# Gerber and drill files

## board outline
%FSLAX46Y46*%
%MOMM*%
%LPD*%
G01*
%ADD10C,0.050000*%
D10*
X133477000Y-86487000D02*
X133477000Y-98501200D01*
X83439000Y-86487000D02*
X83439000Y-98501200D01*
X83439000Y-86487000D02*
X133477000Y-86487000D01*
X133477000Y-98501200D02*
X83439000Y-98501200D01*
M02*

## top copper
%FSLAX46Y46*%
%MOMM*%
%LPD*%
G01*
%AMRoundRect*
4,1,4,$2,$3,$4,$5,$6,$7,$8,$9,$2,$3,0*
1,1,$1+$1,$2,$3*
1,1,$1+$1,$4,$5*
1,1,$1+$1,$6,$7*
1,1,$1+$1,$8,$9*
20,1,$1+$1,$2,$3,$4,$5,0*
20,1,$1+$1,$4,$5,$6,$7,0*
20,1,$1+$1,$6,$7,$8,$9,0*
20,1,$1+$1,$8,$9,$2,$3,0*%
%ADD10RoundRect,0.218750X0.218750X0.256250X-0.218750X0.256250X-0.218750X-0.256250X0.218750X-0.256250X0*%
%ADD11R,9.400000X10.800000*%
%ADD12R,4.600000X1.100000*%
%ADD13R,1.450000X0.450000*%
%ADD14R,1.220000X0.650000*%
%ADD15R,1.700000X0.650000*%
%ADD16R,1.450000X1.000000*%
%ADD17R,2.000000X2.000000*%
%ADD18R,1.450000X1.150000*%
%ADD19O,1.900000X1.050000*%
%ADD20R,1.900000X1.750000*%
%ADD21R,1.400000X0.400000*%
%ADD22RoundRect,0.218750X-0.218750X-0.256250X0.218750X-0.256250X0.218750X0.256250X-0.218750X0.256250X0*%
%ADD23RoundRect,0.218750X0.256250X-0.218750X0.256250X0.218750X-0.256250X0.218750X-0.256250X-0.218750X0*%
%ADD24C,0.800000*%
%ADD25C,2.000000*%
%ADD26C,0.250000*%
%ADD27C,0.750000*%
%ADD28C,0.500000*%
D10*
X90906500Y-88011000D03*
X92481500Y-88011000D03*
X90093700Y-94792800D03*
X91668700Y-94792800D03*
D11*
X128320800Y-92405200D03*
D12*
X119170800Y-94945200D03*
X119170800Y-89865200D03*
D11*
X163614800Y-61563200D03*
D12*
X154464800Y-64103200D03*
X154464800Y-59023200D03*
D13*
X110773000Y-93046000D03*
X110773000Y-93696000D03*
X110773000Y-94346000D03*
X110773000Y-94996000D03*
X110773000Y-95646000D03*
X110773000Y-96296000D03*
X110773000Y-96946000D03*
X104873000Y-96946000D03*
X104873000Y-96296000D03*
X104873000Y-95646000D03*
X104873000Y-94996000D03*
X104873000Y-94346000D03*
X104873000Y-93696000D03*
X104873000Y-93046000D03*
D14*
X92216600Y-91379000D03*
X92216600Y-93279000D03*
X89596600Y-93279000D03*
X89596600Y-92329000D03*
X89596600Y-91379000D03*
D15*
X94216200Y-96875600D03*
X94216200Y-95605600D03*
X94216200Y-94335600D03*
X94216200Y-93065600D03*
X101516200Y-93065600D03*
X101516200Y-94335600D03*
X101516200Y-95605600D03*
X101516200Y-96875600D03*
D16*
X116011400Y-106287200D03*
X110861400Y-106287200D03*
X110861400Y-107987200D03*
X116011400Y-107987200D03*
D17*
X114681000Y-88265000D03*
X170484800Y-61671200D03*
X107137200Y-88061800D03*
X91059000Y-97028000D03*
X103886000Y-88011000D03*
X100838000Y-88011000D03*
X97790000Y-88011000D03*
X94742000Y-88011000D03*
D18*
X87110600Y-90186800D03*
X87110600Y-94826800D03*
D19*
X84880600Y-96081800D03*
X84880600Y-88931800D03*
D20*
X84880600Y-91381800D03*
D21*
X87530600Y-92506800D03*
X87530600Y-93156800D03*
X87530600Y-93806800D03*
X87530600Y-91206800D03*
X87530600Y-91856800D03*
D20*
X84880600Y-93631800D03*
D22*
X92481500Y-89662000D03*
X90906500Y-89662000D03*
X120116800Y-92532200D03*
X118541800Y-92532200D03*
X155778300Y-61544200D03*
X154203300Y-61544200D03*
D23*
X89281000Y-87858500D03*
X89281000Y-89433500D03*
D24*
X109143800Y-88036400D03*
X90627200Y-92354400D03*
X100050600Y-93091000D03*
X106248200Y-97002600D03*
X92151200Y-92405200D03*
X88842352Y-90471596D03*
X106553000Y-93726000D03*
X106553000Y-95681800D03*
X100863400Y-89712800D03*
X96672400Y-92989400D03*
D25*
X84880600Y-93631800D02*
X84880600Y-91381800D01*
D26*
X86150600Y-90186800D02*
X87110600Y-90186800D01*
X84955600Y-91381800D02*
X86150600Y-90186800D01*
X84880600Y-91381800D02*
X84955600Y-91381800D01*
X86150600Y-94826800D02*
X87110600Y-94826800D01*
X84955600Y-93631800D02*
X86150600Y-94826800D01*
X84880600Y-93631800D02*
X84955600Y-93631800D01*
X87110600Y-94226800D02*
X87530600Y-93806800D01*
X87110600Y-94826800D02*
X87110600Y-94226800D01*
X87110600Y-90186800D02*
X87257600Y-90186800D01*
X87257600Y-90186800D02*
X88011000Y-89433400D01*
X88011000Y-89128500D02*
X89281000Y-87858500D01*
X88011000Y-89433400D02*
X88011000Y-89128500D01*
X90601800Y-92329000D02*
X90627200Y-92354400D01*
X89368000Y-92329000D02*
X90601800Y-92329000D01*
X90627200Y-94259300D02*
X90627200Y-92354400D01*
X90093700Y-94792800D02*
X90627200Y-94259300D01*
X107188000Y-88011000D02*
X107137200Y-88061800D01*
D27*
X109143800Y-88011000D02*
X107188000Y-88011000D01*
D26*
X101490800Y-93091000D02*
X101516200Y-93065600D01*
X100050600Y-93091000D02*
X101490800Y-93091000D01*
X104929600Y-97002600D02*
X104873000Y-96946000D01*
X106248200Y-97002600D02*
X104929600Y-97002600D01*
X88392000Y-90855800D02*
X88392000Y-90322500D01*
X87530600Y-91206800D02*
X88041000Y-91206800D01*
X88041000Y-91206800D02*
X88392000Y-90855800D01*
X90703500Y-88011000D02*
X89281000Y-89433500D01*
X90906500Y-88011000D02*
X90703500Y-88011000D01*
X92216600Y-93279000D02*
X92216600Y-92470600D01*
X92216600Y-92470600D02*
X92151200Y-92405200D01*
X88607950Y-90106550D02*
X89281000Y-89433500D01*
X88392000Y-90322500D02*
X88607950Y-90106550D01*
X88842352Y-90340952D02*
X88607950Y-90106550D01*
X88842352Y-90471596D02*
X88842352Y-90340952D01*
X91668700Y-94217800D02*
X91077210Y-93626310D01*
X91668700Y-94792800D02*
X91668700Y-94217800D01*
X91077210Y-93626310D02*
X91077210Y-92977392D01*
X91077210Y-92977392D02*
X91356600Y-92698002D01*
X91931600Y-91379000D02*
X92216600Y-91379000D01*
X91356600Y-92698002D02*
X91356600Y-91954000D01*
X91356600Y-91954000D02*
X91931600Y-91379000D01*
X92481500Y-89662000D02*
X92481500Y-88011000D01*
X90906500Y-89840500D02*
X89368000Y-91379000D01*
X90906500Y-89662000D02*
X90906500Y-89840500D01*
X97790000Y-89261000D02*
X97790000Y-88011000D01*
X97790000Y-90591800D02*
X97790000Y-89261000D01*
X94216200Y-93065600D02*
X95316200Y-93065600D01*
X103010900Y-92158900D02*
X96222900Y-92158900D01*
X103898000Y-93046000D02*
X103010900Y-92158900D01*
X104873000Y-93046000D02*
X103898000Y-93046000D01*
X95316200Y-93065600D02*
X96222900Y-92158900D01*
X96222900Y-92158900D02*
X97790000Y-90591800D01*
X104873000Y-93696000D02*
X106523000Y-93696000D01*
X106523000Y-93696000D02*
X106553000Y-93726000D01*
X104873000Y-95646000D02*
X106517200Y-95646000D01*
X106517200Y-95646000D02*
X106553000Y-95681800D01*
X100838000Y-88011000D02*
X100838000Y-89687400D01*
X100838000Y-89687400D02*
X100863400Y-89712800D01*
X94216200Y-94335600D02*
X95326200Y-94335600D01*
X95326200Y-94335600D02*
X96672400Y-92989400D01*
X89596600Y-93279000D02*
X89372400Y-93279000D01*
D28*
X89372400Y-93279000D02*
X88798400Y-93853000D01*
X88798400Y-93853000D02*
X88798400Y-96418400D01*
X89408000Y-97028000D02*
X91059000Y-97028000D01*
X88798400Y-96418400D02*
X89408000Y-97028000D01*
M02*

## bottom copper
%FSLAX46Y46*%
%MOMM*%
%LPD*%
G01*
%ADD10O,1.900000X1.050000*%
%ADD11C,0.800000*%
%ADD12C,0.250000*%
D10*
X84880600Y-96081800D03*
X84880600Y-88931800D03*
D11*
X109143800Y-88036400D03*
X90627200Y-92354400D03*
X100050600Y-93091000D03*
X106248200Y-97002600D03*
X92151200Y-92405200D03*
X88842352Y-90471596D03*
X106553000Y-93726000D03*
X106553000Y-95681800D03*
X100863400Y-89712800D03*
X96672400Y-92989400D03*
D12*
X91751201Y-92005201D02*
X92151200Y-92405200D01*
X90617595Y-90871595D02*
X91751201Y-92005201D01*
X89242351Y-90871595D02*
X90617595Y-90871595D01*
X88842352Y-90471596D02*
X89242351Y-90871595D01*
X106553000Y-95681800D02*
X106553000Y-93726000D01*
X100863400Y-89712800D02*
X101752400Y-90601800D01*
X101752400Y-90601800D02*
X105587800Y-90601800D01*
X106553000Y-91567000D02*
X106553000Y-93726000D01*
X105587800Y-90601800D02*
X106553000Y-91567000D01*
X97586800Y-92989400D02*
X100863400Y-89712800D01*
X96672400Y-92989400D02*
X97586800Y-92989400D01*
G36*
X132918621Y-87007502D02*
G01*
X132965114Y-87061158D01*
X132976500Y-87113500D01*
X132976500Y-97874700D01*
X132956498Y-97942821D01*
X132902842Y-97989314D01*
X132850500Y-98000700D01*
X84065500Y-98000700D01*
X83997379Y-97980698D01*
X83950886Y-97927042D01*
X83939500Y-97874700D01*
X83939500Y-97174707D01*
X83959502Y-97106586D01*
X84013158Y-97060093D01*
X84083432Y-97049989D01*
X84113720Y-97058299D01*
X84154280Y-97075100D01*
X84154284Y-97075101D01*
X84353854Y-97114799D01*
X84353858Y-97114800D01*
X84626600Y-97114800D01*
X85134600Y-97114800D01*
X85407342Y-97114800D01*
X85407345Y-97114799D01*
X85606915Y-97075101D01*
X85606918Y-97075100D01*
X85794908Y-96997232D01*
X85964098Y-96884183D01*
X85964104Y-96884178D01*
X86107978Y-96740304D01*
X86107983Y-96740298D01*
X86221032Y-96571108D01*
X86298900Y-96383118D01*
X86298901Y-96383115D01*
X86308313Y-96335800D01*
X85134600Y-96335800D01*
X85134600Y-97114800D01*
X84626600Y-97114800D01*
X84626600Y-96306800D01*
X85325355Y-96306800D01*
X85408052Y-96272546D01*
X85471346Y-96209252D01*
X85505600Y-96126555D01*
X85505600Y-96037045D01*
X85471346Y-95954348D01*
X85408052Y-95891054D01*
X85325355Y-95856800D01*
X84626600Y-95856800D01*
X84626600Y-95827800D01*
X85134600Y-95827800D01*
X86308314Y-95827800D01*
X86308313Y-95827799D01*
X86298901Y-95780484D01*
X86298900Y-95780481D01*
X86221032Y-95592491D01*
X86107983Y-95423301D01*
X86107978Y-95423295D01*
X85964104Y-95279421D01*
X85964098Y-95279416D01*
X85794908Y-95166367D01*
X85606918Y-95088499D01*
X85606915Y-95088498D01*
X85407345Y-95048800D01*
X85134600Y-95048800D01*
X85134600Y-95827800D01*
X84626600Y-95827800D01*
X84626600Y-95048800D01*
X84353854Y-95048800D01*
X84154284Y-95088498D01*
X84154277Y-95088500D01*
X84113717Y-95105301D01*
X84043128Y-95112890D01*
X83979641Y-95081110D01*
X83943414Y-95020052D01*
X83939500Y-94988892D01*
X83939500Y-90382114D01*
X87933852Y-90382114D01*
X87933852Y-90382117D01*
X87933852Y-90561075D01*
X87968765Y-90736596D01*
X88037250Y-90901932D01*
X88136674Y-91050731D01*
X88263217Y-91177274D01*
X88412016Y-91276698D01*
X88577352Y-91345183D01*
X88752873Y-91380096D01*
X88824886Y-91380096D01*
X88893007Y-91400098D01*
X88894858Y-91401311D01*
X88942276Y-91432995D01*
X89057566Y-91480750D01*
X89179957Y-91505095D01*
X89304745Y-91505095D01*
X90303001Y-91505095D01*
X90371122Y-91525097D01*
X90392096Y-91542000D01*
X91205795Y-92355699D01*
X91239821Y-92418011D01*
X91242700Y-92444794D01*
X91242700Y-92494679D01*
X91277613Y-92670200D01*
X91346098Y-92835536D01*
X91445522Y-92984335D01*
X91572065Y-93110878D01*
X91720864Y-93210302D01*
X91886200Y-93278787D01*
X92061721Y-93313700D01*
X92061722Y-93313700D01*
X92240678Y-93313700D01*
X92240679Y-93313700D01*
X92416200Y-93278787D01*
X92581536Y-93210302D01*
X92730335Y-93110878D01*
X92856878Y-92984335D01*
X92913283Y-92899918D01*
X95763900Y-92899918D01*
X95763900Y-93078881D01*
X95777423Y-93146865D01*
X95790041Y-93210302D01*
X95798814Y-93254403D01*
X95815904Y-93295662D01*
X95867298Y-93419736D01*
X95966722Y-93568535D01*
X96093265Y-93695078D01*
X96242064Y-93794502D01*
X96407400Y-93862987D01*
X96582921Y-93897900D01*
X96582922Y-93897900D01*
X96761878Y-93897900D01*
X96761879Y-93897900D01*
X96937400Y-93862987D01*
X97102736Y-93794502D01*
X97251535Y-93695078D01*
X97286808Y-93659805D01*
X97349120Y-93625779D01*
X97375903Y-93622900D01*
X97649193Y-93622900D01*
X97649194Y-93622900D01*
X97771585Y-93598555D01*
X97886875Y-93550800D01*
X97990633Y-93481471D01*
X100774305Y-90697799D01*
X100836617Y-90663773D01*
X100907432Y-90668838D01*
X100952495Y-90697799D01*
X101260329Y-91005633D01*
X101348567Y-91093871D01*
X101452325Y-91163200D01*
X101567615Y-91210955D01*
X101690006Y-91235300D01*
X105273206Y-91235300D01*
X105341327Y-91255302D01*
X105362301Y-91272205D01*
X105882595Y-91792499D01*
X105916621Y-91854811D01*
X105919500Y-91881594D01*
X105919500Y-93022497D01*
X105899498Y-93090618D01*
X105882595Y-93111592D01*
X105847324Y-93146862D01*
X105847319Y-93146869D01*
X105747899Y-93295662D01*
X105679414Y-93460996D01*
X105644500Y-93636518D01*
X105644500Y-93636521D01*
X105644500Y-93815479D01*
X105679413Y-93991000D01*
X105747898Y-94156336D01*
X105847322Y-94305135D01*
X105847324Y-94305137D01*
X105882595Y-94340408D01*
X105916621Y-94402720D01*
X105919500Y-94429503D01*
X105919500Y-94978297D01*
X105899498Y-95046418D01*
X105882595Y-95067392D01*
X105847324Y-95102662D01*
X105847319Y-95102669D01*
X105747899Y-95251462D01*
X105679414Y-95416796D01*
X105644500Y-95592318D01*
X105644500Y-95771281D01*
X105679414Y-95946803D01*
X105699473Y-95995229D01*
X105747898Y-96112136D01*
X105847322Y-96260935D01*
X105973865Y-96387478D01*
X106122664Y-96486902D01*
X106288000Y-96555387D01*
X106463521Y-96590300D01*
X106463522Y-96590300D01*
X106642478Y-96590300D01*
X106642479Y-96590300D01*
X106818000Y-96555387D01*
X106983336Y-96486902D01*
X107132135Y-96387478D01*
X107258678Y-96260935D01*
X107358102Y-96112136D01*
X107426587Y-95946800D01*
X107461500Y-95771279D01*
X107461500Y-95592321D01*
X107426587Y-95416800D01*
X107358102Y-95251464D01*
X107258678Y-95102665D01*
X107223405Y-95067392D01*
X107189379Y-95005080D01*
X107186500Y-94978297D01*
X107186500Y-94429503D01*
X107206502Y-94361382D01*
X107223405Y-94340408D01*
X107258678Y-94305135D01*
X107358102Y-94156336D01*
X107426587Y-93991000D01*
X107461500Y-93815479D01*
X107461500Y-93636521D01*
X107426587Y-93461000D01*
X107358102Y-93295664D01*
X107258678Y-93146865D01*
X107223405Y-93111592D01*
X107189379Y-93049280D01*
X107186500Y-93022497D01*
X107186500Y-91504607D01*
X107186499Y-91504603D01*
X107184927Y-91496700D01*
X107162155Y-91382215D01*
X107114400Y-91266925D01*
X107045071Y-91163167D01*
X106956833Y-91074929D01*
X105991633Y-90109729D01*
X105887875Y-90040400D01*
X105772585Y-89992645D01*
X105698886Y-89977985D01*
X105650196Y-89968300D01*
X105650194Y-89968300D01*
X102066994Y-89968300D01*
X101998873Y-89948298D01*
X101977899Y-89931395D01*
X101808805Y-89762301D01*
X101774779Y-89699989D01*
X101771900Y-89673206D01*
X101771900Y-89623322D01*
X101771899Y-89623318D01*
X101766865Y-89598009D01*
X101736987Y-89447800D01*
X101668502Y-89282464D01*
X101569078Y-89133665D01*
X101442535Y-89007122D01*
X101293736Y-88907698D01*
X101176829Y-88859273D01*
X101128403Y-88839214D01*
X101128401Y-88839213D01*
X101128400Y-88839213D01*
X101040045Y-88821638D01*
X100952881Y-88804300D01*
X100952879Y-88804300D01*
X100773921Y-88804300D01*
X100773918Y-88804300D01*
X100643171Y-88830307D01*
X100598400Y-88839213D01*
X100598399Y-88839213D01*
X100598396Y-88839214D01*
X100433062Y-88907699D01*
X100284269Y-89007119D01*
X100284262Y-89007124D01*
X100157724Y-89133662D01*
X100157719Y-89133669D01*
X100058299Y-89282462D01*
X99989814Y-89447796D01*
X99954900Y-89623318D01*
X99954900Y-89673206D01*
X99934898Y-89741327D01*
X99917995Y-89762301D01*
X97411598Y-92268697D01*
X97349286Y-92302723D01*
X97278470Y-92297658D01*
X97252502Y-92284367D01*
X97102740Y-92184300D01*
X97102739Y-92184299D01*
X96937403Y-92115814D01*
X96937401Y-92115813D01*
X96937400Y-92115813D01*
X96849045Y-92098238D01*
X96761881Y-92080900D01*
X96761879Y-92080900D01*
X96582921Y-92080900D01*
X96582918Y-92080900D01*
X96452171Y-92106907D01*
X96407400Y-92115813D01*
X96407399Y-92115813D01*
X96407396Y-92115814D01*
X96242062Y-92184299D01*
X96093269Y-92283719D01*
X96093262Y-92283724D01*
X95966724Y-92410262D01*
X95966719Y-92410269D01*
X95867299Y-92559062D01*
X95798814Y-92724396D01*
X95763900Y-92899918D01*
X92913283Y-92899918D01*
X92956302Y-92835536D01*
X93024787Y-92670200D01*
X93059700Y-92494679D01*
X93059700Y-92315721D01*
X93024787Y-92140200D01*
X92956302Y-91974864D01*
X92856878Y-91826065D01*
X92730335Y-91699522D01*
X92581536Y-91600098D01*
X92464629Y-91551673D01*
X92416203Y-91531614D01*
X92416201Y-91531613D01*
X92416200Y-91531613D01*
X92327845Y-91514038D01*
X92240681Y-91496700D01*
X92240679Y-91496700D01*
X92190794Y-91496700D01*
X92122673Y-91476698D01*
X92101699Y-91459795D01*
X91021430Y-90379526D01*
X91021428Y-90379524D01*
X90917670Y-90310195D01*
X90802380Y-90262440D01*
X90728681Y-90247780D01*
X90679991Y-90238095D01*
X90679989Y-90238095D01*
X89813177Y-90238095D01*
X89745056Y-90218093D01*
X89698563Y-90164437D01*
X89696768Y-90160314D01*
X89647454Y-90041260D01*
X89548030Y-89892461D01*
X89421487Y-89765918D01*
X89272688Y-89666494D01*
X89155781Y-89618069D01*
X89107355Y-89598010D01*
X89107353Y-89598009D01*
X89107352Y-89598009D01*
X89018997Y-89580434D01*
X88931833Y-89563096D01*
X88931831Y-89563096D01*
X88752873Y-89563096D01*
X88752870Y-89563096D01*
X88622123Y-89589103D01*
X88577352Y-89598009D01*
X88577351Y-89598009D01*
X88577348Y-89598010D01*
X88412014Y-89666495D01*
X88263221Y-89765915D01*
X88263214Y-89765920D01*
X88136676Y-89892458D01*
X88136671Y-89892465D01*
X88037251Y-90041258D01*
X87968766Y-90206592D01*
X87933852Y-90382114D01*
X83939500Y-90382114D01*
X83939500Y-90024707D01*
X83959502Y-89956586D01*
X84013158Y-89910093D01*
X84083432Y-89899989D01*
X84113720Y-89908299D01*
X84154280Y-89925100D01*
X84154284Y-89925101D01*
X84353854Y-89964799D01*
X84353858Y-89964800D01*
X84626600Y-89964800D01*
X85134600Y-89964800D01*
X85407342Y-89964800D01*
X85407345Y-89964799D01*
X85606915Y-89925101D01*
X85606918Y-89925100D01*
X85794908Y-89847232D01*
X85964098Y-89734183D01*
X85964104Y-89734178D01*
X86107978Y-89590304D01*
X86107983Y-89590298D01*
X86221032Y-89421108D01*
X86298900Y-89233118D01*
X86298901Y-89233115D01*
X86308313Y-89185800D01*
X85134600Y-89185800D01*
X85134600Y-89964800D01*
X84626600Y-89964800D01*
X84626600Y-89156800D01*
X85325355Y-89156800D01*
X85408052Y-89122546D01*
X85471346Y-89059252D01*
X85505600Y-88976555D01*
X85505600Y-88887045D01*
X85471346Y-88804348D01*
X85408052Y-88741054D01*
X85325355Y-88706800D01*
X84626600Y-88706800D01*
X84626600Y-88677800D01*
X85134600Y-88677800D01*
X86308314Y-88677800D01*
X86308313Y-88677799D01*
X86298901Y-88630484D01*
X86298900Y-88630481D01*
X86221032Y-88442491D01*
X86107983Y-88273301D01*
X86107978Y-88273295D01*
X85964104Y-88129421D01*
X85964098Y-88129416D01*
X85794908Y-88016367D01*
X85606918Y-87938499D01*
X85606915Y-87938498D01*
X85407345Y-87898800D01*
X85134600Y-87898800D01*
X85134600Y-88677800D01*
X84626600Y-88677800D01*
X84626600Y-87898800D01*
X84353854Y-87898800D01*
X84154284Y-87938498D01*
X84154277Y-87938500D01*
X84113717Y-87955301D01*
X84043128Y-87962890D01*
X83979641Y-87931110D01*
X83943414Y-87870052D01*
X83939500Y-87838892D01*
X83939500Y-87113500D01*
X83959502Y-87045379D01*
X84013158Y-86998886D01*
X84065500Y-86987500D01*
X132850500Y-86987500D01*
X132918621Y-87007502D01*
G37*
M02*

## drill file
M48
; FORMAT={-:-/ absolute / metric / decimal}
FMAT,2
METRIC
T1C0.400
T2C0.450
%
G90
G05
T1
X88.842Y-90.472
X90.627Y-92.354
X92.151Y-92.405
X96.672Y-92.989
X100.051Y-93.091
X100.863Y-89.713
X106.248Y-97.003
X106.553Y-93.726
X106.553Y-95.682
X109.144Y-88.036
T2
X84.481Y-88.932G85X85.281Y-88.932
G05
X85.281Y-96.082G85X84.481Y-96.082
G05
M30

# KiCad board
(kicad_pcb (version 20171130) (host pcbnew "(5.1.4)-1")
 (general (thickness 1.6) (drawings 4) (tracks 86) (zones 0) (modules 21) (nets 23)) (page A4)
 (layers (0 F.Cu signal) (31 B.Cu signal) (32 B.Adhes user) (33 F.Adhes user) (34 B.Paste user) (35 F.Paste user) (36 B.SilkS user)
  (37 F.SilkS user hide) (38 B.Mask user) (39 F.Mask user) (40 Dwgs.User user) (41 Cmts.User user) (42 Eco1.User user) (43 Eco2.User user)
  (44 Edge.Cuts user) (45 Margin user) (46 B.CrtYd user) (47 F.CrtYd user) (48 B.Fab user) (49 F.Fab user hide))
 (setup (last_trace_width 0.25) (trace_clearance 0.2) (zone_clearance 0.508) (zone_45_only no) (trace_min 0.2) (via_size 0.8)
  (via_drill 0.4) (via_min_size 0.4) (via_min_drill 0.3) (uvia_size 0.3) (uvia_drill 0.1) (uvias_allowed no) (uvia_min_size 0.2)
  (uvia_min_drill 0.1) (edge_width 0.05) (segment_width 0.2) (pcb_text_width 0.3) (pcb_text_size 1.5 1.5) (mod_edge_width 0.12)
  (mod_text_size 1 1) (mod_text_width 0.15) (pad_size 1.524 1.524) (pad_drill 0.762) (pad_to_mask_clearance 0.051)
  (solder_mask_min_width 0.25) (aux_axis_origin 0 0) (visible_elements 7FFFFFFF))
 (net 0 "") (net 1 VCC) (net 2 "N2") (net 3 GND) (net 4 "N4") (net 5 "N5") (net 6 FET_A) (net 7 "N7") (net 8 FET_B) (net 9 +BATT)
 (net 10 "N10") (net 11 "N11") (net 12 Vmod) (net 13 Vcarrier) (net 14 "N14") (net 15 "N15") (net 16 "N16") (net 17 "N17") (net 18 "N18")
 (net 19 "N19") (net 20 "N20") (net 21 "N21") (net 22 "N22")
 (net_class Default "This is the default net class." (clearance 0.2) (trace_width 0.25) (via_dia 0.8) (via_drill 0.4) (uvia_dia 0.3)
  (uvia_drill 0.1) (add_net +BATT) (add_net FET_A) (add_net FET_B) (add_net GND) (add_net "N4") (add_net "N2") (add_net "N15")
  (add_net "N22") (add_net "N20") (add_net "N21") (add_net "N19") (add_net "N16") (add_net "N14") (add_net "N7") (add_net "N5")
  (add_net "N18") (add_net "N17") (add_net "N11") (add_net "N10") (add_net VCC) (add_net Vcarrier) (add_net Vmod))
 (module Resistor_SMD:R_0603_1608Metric (layer F.Cu) (at 91.694 88.011 180)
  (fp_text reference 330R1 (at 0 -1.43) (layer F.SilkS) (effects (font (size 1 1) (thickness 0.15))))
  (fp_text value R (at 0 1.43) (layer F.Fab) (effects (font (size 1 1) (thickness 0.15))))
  (pad 2 smd roundrect (at 0.7875 0 180) (size 0.875 0.95) (layers F.Cu F.Paste F.Mask) (roundrect_rratio 0.25) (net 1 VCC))
  (pad 1 smd roundrect (at -0.7875 0 180) (size 0.875 0.95) (layers F.Cu F.Paste F.Mask) (roundrect_rratio 0.25) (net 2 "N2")))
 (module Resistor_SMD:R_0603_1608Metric (layer F.Cu) (at 90.8812 94.7928 180)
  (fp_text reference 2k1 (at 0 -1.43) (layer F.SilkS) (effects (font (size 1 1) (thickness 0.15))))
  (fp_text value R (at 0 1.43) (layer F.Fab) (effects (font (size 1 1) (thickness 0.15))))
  (pad 2 smd roundrect (at 0.7875 0 180) (size 0.875 0.95) (layers F.Cu F.Paste F.Mask) (roundrect_rratio 0.25) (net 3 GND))
  (pad 1 smd roundrect (at -0.7875 0 180) (size 0.875 0.95) (layers F.Cu F.Paste F.Mask) (roundrect_rratio 0.25) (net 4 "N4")))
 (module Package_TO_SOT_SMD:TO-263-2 (layer F.Cu) (at 124.9458 92.4052)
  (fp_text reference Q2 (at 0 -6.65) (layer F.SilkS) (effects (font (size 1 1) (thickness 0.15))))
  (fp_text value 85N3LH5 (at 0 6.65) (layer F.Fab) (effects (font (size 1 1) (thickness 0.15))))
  (pad "" smd rect (at 0.95 2.775) (size 4.55 5.25) (layers F.Paste))
  (pad "" smd rect (at 5.8 -2.775) (size 4.55 5.25) (layers F.Paste))
  (pad "" smd rect (at 0.95 -2.775) (size 4.55 5.25) (layers F.Paste))
  (pad "" smd rect (at 5.8 2.775) (size 4.55 5.25) (layers F.Paste))
  (pad 2 smd rect (at 3.375 0) (size 9.4 10.8) (layers F.Cu F.Mask) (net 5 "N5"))
  (pad 3 smd rect (at -5.775 2.54) (size 4.6 1.1) (layers F.Cu F.Paste F.Mask) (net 3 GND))
  (pad 1 smd rect (at -5.775 -2.54) (size 4.6 1.1) (layers F.Cu F.Paste F.Mask) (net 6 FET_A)))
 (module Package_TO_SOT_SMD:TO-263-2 (layer F.Cu) (at 160.2398 61.5632)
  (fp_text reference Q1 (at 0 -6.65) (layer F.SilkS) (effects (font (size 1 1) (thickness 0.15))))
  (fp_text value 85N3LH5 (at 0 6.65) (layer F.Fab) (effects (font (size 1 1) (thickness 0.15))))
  (pad "" smd rect (at 0.95 2.775) (size 4.55 5.25) (layers F.Paste))
  (pad "" smd rect (at 5.8 -2.775) (size 4.55 5.25) (layers F.Paste))
  (pad "" smd rect (at 0.95 -2.775) (size 4.55 5.25) (layers F.Paste))
  (pad "" smd rect (at 5.8 2.775) (size 4.55 5.25) (layers F.Paste))
  (pad 2 smd rect (at 3.375 0) (size 9.4 10.8) (layers F.Cu F.Mask) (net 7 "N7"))
  (pad 3 smd rect (at -5.775 2.54) (size 4.6 1.1) (layers F.Cu F.Paste F.Mask) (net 3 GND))
  (pad 1 smd rect (at -5.775 -2.54) (size 4.6 1.1) (layers F.Cu F.Paste F.Mask) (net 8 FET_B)))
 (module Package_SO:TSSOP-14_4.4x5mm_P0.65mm (layer F.Cu) (at 107.823 94.996)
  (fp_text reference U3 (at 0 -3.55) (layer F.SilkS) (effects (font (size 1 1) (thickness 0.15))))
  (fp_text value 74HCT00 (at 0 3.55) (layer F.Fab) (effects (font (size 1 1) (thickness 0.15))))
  (pad 14 smd rect (at 2.95 -1.95) (size 1.45 0.45) (layers F.Cu F.Paste F.Mask) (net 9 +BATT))
  (pad 13 smd rect (at 2.95 -1.3) (size 1.45 0.45) (layers F.Cu F.Paste F.Mask) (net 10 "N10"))
  (pad 12 smd rect (at 2.95 -0.65) (size 1.45 0.45) (layers F.Cu F.Paste F.Mask) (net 10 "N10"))
  (pad 11 smd rect (at 2.95 0) (size 1.45 0.45) (layers F.Cu F.Paste F.Mask) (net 8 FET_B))
  (pad 10 smd rect (at 2.95 0.65) (size 1.45 0.45) (layers F.Cu F.Paste F.Mask) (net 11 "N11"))
  (pad 9 smd rect (at 2.95 1.3) (size 1.45 0.45) (layers F.Cu F.Paste F.Mask) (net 11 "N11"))
  (pad 8 smd rect (at 2.95 1.95) (size 1.45 0.45) (layers F.Cu F.Paste F.Mask) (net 6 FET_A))
  (pad 7 smd rect (at -2.95 1.95) (size 1.45 0.45) (layers F.Cu F.Paste F.Mask) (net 3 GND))
  (pad 6 smd rect (at -2.95 1.3) (size 1.45 0.45) (layers F.Cu F.Paste F.Mask) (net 11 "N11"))
  (pad 5 smd rect (at -2.95 0.65) (size 1.45 0.45) (layers F.Cu F.Paste F.Mask) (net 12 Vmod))
  (pad 4 smd rect (at -2.95 0) (size 1.45 0.45) (layers F.Cu F.Paste F.Mask) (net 10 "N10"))
  (pad 3 smd rect (at -2.95 -0.65) (size 1.45 0.45) (layers F.Cu F.Paste F.Mask) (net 10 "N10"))
  (pad 2 smd rect (at -2.95 -1.3) (size 1.45 0.45) (layers F.Cu F.Paste F.Mask) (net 12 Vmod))
  (pad 1 smd rect (at -2.95 -1.95) (size 1.45 0.45) (layers F.Cu F.Paste F.Mask) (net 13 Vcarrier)))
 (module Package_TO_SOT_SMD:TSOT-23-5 (layer F.Cu) (at 90.9066 92.329)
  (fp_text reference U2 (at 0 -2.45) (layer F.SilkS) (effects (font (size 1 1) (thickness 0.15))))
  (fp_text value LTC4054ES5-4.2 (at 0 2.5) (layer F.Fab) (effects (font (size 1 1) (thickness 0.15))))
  (pad 5 smd rect (at 1.31 -0.95) (size 1.22 0.65) (layers F.Cu F.Paste F.Mask) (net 4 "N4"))
  (pad 4 smd rect (at 1.31 0.95) (size 1.22 0.65) (layers F.Cu F.Paste F.Mask) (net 1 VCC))
  (pad 3 smd rect (at -1.31 0.95) (size 1.22 0.65) (layers F.Cu F.Paste F.Mask) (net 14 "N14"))
  (pad 2 smd rect (at -1.31 0) (size 1.22 0.65) (layers F.Cu F.Paste F.Mask) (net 3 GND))
  (pad 1 smd rect (at -1.31 -0.95) (size 1.22 0.65) (layers F.Cu F.Paste F.Mask) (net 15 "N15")))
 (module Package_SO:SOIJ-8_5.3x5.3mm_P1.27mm (layer F.Cu) (at 97.8662 94.9706 180)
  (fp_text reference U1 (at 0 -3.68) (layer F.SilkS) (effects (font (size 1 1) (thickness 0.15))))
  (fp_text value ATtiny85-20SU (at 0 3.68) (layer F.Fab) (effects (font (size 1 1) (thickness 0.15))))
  (pad 8 smd rect (at 3.65 -1.905 180) (size 1.7 0.65) (layers F.Cu F.Paste F.Mask) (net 9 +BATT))
  (pad 7 smd rect (at 3.65 -0.635 180) (size 1.7 0.65) (layers F.Cu F.Paste F.Mask) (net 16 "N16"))
  (pad 6 smd rect (at 3.65 0.635 180) (size 1.7 0.65) (layers F.Cu F.Paste F.Mask) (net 12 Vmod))
  (pad 5 smd rect (at 3.65 1.905 180) (size 1.7 0.65) (layers F.Cu F.Paste F.Mask) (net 13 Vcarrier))
  (pad 4 smd rect (at -3.65 1.905 180) (size 1.7 0.65) (layers F.Cu F.Paste F.Mask) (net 3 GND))
  (pad 3 smd rect (at -3.65 0.635 180) (size 1.7 0.65) (layers F.Cu F.Paste F.Mask) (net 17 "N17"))
  (pad 2 smd rect (at -3.65 -0.635 180) (size 1.7 0.65) (layers F.Cu F.Paste F.Mask) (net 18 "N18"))
  (pad 1 smd rect (at -3.65 -1.905 180) (size 1.7 0.65) (layers F.Cu F.Paste F.Mask) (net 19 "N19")))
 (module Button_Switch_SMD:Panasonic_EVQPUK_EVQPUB (layer F.Cu) (at 113.4364 107.1372)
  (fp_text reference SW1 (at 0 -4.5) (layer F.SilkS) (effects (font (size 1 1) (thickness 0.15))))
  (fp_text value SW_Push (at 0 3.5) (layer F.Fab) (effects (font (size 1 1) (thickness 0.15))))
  (pad 1 smd rect (at 2.575 -0.85 180) (size 1.45 1) (layers F.Cu F.Paste F.Mask) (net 14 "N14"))
  (pad 1 smd rect (at -2.575 -0.85 180) (size 1.45 1) (layers F.Cu F.Paste F.Mask) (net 14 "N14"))
  (pad 2 smd rect (at -2.575 0.85 180) (size 1.45 1) (layers F.Cu F.Paste F.Mask) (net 9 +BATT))
  (pad 2 smd rect (at 2.575 0.85 180) (size 1.45 1) (layers F.Cu F.Paste F.Mask) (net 9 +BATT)))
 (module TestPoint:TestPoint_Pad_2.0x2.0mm (layer F.Cu) (at 114.681 88.265)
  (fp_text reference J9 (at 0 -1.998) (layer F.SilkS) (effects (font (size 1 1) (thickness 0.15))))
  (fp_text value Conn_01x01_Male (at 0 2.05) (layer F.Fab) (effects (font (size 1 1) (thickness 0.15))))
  (pad 1 smd rect (at 0 0) (size 2 2) (layers F.Cu F.Mask) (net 5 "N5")))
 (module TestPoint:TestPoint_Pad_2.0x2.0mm (layer F.Cu) (at 170.4848 61.6712)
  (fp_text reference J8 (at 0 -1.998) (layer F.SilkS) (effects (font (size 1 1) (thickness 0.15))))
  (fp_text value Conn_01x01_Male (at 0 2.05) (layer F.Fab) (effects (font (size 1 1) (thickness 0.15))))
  (pad 1 smd rect (at 0 0) (size 2 2) (layers F.Cu F.Mask) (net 7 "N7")))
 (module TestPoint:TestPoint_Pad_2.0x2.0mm (layer F.Cu) (at 107.1372 88.0618)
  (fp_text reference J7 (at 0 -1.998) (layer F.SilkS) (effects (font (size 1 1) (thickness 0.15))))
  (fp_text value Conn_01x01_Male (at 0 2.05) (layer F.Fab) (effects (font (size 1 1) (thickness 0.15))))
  (pad 1 smd rect (at 0 0) (size 2 2) (layers F.Cu F.Mask) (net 3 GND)))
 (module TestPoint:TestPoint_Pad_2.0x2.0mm (layer F.Cu) (at 91.059 97.028)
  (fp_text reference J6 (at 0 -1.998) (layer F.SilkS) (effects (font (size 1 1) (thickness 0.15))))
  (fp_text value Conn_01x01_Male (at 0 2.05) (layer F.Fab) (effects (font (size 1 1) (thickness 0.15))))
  (pad 1 smd rect (at 0 0) (size 2 2) (layers F.Cu F.Mask) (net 14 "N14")))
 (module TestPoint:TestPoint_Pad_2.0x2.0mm (layer F.Cu) (at 103.886 88.011)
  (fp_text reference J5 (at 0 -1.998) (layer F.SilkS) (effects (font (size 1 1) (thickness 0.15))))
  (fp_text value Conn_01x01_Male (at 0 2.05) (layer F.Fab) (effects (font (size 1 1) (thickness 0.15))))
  (pad 1 smd rect (at 0 0) (size 2 2) (layers F.Cu F.Mask) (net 16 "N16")))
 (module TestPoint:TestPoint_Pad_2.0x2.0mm (layer F.Cu) (at 100.838 88.011)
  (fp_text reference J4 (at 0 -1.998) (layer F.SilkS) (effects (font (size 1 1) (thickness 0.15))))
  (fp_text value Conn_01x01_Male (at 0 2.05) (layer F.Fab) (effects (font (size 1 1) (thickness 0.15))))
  (pad 1 smd rect (at 0 0) (size 2 2) (layers F.Cu F.Mask) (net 12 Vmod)))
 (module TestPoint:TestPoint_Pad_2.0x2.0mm (layer F.Cu) (at 97.79 88.011)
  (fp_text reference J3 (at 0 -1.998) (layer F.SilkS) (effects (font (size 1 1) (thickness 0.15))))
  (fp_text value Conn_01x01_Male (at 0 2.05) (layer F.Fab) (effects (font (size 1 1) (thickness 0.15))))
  (pad 1 smd rect (at 0 0) (size 2 2) (layers F.Cu F.Mask) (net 13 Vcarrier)))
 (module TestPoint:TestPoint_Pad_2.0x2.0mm (layer F.Cu) (at 94.742 88.011)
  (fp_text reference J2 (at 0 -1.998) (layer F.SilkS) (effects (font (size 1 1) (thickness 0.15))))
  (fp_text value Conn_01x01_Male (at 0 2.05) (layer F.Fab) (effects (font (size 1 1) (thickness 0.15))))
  (pad 1 smd rect (at 0 0) (size 2 2) (layers F.Cu F.Mask) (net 19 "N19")))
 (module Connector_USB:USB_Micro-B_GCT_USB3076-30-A (layer F.Cu) (at 86.0806 92.5068 270)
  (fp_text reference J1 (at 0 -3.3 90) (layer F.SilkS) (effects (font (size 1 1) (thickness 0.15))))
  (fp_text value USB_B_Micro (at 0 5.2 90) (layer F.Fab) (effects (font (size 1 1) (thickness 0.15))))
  (pad 6 smd rect (at -2.32 -1.03 270) (size 1.15 1.45) (layers F.Cu F.Paste F.Mask) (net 3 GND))
  (pad 6 smd rect (at 2.32 -1.03 270) (size 1.15 1.45) (layers F.Cu F.Paste F.Mask) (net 3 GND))
  (pad 6 thru_hole oval (at 3.575 1.2 270) (size 1.05 1.9) (drill oval 0.45 1.25) (layers *.Cu *.Mask) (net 3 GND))
  (pad 6 thru_hole oval (at -3.575 1.2 90) (size 1.05 1.9) (drill oval 0.45 1.25) (layers *.Cu *.Mask) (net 3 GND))
  (pad 6 smd rect (at -1.125 1.2 270) (size 1.75 1.9) (layers F.Cu F.Paste F.Mask) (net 3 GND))
  (pad 3 smd rect (at 0 -1.45 270) (size 0.4 1.4) (layers F.Cu F.Paste F.Mask) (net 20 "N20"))
  (pad 4 smd rect (at 0.65 -1.45 270) (size 0.4 1.4) (layers F.Cu F.Paste F.Mask) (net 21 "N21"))
  (pad 5 smd rect (at 1.3 -1.45 270) (size 0.4 1.4) (layers F.Cu F.Paste F.Mask) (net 3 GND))
  (pad 1 smd rect (at -1.3 -1.45 270) (size 0.4 1.4) (layers F.Cu F.Paste F.Mask) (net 1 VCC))
  (pad 2 smd rect (at -0.65 -1.45 270) (size 0.4 1.4) (layers F.Cu F.Paste F.Mask) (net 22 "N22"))
  (pad 6 smd rect (at 1.125 1.2 270) (size 1.75 1.9) (layers F.Cu F.Paste F.Mask) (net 3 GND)))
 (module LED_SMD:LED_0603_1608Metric (layer F.Cu) (at 91.694 89.662)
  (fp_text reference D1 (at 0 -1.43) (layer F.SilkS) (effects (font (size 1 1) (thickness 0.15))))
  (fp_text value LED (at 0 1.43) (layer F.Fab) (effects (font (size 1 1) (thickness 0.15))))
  (pad 2 smd roundrect (at 0.7875 0) (size 0.875 0.95) (layers F.Cu F.Paste F.Mask) (roundrect_rratio 0.25) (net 2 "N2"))
  (pad 1 smd roundrect (at -0.7875 0) (size 0.875 0.95) (layers F.Cu F.Paste F.Mask) (roundrect_rratio 0.25) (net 15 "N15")))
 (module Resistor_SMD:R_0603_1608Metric (layer F.Cu) (at 119.3293 92.5322)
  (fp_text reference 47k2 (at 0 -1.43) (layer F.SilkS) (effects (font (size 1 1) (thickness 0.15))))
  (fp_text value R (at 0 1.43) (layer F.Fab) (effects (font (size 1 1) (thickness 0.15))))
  (pad 2 smd roundrect (at 0.7875 0) (size 0.875 0.95) (layers F.Cu F.Paste F.Mask) (roundrect_rratio 0.25) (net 6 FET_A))
  (pad 1 smd roundrect (at -0.7875 0) (size 0.875 0.95) (layers F.Cu F.Paste F.Mask) (roundrect_rratio 0.25) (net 3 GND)))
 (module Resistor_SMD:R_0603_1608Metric (layer F.Cu) (at 154.9908 61.5442)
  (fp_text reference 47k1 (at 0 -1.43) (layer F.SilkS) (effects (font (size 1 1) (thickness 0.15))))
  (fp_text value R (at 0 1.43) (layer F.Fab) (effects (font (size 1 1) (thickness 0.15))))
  (pad 2 smd roundrect (at 0.7875 0) (size 0.875 0.95) (layers F.Cu F.Paste F.Mask) (roundrect_rratio 0.25) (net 8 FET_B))
  (pad 1 smd roundrect (at -0.7875 0) (size 0.875 0.95) (layers F.Cu F.Paste F.Mask) (roundrect_rratio 0.25) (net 3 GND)))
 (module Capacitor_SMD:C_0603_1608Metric (layer F.Cu) (at 89.281 88.646 90)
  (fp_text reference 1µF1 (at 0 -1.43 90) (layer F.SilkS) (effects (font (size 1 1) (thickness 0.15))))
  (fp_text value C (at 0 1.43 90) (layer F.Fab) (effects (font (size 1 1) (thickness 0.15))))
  (pad 2 smd roundrect (at 0.7875 0 90) (size 0.875 0.95) (layers F.Cu F.Paste F.Mask) (roundrect_rratio 0.25) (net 3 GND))
  (pad 1 smd roundrect (at -0.7875 0 90) (size 0.875 0.95) (layers F.Cu F.Paste F.Mask) (roundrect_rratio 0.25) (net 1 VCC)))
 (gr_line (start 133.477 86.487) (end 133.477 98.5012) (layer Edge.Cuts) (width 0.05))
 (gr_line (start 83.439 86.487) (end 83.439 98.5012) (layer Edge.Cuts) (width 0.05))
 (gr_line (start 83.439 86.487) (end 133.477 86.487) (layer Edge.Cuts) (width 0.05))
 (gr_line (start 133.477 98.5012) (end 83.439 98.5012) (layer Edge.Cuts) (width 0.05))
 (via (at 109.1438 88.0364) (size 0.8) (drill 0.4) (layers F.Cu B.Cu) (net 3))
 (segment (start 84.8806 93.6318) (end 84.8806 91.3818) (width 2) (layer F.Cu) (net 3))
 (segment (start 86.1506 90.1868) (end 87.1106 90.1868) (width 0.25) (layer F.Cu) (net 3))
 (segment (start 84.9556 91.3818) (end 86.1506 90.1868) (width 0.25) (layer F.Cu) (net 3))
 (segment (start 84.8806 91.3818) (end 84.9556 91.3818) (width 0.25) (layer F.Cu) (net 3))
 (segment (start 86.1506 94.8268) (end 87.1106 94.8268) (width 0.25) (layer F.Cu) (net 3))
 (segment (start 84.9556 93.6318) (end 86.1506 94.8268) (width 0.25) (layer F.Cu) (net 3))
 (segment (start 84.8806 93.6318) (end 84.9556 93.6318) (width 0.25) (layer F.Cu) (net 3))
 (segment (start 87.1106 94.2268) (end 87.5306 93.8068) (width 0.25) (layer F.Cu) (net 3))
 (segment (start 87.1106 94.8268) (end 87.1106 94.2268) (width 0.25) (layer F.Cu) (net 3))
 (segment (start 87.1106 90.1868) (end 87.2576 90.1868) (width 0.25) (layer F.Cu) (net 3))
 (segment (start 87.2576 90.1868) (end 88.011 89.4334) (width 0.25) (layer F.Cu) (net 3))
 (segment (start 88.011 89.1285) (end 89.281 87.8585) (width 0.25) (layer F.Cu) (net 3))
 (segment (start 88.011 89.4334) (end 88.011 89.1285) (width 0.25) (layer F.Cu) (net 3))
 (via (at 90.6272 92.3544) (size 0.8) (drill 0.4) (layers F.Cu B.Cu) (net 3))
 (segment (start 90.6018 92.329) (end 90.6272 92.3544) (width 0.25) (layer F.Cu) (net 3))
 (segment (start 89.368 92.329) (end 90.6018 92.329) (width 0.25) (layer F.Cu) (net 3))
 (segment (start 90.6272 94.2593) (end 90.6272 92.3544) (width 0.25) (layer F.Cu) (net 3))
 (segment (start 90.0937 94.7928) (end 90.6272 94.2593) (width 0.25) (layer F.Cu) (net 3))
 (segment (start 107.188 88.011) (end 107.1372 88.0618) (width 0.25) (layer F.Cu) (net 3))
 (segment (start 109.1438 88.011) (end 107.188 88.011) (width 0.75) (layer F.Cu) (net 3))
 (via (at 100.0506 93.091) (size 0.8) (drill 0.4) (layers F.Cu B.Cu) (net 3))
 (segment (start 101.4908 93.091) (end 101.5162 93.0656) (width 0.25) (layer F.Cu) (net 3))
 (segment (start 100.0506 93.091) (end 101.4908 93.091) (width 0.25) (layer F.Cu) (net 3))
 (via (at 106.2482 97.0026) (size 0.8) (drill 0.4) (layers F.Cu B.Cu) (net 3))
 (segment (start 104.9296 97.0026) (end 104.873 96.946) (width 0.25) (layer F.Cu) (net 3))
 (segment (start 106.2482 97.0026) (end 104.9296 97.0026) (width 0.25) (layer F.Cu) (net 3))
 (segment (start 88.392 90.8558) (end 88.392 90.3225) (width 0.25) (layer F.Cu) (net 1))
 (segment (start 87.5306 91.2068) (end 88.041 91.2068) (width 0.25) (layer F.Cu) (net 1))
 (segment (start 88.041 91.2068) (end 88.392 90.8558) (width 0.25) (layer F.Cu) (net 1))
 (segment (start 90.7035 88.011) (end 89.281 89.4335) (width 0.25) (layer F.Cu) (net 1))
 (segment (start 90.9065 88.011) (end 90.7035 88.011) (width 0.25) (layer F.Cu) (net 1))
 (via (at 92.1512 92.4052) (size 0.8) (drill 0.4) (layers F.Cu B.Cu) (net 1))
 (segment (start 92.2166 93.279) (end 92.2166 92.4706) (width 0.25) (layer F.Cu) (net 1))
 (segment (start 92.2166 92.4706) (end 92.1512 92.4052) (width 0.25) (layer F.Cu) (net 1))
 (via (at 88.842352 90.471596) (size 0.8) (drill 0.4) (layers F.Cu B.Cu) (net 1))
 (segment (start 88.60795 90.10655) (end 89.281 89.4335) (width 0.25) (layer F.Cu) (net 1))
 (segment (start 88.392 90.3225) (end 88.60795 90.10655) (width 0.25) (layer F.Cu) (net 1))
 (segment (start 91.751201 92.005201) (end 92.1512 92.4052) (width 0.25) (layer B.Cu) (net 1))
 (segment (start 90.617595 90.871595) (end 91.751201 92.005201) (width 0.25) (layer B.Cu) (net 1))
 (segment (start 89.242351 90.871595) (end 90.617595 90.871595) (width 0.25) (layer B.Cu) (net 1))
 (segment (start 88.842352 90.471596) (end 89.242351 90.871595) (width 0.25) (layer B.Cu) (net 1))
 (segment (start 88.842352 90.340952) (end 88.60795 90.10655) (width 0.25) (layer F.Cu) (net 1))
 (segment (start 88.842352 90.471596) (end 88.842352 90.340952) (width 0.25) (layer F.Cu) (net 1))
 (segment (start 91.6687 94.2178) (end 91.07721 93.62631) (width 0.25) (layer F.Cu) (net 4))
 (segment (start 91.6687 94.7928) (end 91.6687 94.2178) (width 0.25) (layer F.Cu) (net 4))
 (segment (start 91.07721 93.62631) (end 91.07721 92.977392) (width 0.25) (layer F.Cu) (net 4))
 (segment (start 91.07721 92.977392) (end 91.3566 92.698002) (width 0.25) (layer F.Cu) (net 4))
 (segment (start 91.9316 91.379) (end 92.2166 91.379) (width 0.25) (layer F.Cu) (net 4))
 (segment (start 91.3566 92.698002) (end 91.3566 91.954) (width 0.25) (layer F.Cu) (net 4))
 (segment (start 91.3566 91.954) (end 91.9316 91.379) (width 0.25) (layer F.Cu) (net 4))
 (segment (start 92.4815 89.662) (end 92.4815 88.011) (width 0.25) (layer F.Cu) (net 2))
 (segment (start 90.9065 89.8405) (end 89.368 91.379) (width 0.25) (layer F.Cu) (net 15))
 (segment (start 90.9065 89.662) (end 90.9065 89.8405) (width 0.25) (layer F.Cu) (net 15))
 (segment (start 97.79 89.261) (end 97.79 88.011) (width 0.25) (layer F.Cu) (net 13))
 (segment (start 97.79 90.5918) (end 97.79 89.261) (width 0.25) (layer F.Cu) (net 13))
 (segment (start 94.2162 93.0656) (end 95.3162 93.0656) (width 0.25) (layer F.Cu) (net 13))
 (segment (start 103.0109 92.1589) (end 96.2229 92.1589) (width 0.25) (layer F.Cu) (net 13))
 (segment (start 103.898 93.046) (end 103.0109 92.1589) (width 0.25) (layer F.Cu) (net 13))
 (segment (start 104.873 93.046) (end 103.898 93.046) (width 0.25) (layer F.Cu) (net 13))
 (segment (start 95.3162 93.0656) (end 96.2229 92.1589) (width 0.25) (layer F.Cu) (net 13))
 (segment (start 96.2229 92.1589) (end 97.79 90.5918) (width 0.25) (layer F.Cu) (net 13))
 (via (at 106.553 93.726) (size 0.8) (drill 0.4) (layers F.Cu B.Cu) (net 12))
 (segment (start 104.873 93.696) (end 106.523 93.696) (width 0.25) (layer F.Cu) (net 12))
 (segment (start 106.523 93.696) (end 106.553 93.726) (width 0.25) (layer F.Cu) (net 12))
 (via (at 106.553 95.6818) (size 0.8) (drill 0.4) (layers F.Cu B.Cu) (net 12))
 (segment (start 104.873 95.646) (end 106.5172 95.646) (width 0.25) (layer F.Cu) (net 12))
 (segment (start 106.5172 95.646) (end 106.553 95.6818) (width 0.25) (layer F.Cu) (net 12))
 (segment (start 106.553 95.6818) (end 106.553 93.726) (width 0.25) (layer B.Cu) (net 12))
 (via (at 100.8634 89.7128) (size 0.8) (drill 0.4) (layers F.Cu B.Cu) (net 12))
 (segment (start 100.838 88.011) (end 100.838 89.6874) (width 0.25) (layer F.Cu) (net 12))
 (segment (start 100.838 89.6874) (end 100.8634 89.7128) (width 0.25) (layer F.Cu) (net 12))
 (segment (start 100.8634 89.7128) (end 101.7524 90.6018) (width 0.25) (layer B.Cu) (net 12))
 (segment (start 101.7524 90.6018) (end 105.5878 90.6018) (width 0.25) (layer B.Cu) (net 12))
 (segment (start 106.553 91.567) (end 106.553 93.726) (width 0.25) (layer B.Cu) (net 12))
 (segment (start 105.5878 90.6018) (end 106.553 91.567) (width 0.25) (layer B.Cu) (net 12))
 (via (at 96.6724 92.9894) (size 0.8) (drill 0.4) (layers F.Cu B.Cu) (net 12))
 (segment (start 94.2162 94.3356) (end 95.3262 94.3356) (width 0.25) (layer F.Cu) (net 12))
 (segment (start 95.3262 94.3356) (end 96.6724 92.9894) (width 0.25) (layer F.Cu) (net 12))
 (segment (start 97.5868 92.9894) (end 100.8634 89.7128) (width 0.25) (layer B.Cu) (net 12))
 (segment (start 96.6724 92.9894) (end 97.5868 92.9894) (width 0.25) (layer B.Cu) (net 12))
 (segment (start 89.5966 93.279) (end 89.3724 93.279) (width 0.25) (layer F.Cu) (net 14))
 (segment (start 89.3724 93.279) (end 88.7984 93.853) (width 0.5) (layer F.Cu) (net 14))
 (segment (start 88.7984 93.853) (end 88.7984 96.4184) (width 0.5) (layer F.Cu) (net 14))
 (segment (start 89.408 97.028) (end 91.059 97.028) (width 0.5) (layer F.Cu) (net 14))
 (segment (start 88.7984 96.4184) (end 89.408 97.028) (width 0.5) (layer F.Cu) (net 14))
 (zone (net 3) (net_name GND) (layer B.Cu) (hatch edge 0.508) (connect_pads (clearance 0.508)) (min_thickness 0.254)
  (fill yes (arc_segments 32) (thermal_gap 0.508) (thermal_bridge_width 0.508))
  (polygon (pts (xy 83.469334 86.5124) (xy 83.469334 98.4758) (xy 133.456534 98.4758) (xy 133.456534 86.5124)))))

